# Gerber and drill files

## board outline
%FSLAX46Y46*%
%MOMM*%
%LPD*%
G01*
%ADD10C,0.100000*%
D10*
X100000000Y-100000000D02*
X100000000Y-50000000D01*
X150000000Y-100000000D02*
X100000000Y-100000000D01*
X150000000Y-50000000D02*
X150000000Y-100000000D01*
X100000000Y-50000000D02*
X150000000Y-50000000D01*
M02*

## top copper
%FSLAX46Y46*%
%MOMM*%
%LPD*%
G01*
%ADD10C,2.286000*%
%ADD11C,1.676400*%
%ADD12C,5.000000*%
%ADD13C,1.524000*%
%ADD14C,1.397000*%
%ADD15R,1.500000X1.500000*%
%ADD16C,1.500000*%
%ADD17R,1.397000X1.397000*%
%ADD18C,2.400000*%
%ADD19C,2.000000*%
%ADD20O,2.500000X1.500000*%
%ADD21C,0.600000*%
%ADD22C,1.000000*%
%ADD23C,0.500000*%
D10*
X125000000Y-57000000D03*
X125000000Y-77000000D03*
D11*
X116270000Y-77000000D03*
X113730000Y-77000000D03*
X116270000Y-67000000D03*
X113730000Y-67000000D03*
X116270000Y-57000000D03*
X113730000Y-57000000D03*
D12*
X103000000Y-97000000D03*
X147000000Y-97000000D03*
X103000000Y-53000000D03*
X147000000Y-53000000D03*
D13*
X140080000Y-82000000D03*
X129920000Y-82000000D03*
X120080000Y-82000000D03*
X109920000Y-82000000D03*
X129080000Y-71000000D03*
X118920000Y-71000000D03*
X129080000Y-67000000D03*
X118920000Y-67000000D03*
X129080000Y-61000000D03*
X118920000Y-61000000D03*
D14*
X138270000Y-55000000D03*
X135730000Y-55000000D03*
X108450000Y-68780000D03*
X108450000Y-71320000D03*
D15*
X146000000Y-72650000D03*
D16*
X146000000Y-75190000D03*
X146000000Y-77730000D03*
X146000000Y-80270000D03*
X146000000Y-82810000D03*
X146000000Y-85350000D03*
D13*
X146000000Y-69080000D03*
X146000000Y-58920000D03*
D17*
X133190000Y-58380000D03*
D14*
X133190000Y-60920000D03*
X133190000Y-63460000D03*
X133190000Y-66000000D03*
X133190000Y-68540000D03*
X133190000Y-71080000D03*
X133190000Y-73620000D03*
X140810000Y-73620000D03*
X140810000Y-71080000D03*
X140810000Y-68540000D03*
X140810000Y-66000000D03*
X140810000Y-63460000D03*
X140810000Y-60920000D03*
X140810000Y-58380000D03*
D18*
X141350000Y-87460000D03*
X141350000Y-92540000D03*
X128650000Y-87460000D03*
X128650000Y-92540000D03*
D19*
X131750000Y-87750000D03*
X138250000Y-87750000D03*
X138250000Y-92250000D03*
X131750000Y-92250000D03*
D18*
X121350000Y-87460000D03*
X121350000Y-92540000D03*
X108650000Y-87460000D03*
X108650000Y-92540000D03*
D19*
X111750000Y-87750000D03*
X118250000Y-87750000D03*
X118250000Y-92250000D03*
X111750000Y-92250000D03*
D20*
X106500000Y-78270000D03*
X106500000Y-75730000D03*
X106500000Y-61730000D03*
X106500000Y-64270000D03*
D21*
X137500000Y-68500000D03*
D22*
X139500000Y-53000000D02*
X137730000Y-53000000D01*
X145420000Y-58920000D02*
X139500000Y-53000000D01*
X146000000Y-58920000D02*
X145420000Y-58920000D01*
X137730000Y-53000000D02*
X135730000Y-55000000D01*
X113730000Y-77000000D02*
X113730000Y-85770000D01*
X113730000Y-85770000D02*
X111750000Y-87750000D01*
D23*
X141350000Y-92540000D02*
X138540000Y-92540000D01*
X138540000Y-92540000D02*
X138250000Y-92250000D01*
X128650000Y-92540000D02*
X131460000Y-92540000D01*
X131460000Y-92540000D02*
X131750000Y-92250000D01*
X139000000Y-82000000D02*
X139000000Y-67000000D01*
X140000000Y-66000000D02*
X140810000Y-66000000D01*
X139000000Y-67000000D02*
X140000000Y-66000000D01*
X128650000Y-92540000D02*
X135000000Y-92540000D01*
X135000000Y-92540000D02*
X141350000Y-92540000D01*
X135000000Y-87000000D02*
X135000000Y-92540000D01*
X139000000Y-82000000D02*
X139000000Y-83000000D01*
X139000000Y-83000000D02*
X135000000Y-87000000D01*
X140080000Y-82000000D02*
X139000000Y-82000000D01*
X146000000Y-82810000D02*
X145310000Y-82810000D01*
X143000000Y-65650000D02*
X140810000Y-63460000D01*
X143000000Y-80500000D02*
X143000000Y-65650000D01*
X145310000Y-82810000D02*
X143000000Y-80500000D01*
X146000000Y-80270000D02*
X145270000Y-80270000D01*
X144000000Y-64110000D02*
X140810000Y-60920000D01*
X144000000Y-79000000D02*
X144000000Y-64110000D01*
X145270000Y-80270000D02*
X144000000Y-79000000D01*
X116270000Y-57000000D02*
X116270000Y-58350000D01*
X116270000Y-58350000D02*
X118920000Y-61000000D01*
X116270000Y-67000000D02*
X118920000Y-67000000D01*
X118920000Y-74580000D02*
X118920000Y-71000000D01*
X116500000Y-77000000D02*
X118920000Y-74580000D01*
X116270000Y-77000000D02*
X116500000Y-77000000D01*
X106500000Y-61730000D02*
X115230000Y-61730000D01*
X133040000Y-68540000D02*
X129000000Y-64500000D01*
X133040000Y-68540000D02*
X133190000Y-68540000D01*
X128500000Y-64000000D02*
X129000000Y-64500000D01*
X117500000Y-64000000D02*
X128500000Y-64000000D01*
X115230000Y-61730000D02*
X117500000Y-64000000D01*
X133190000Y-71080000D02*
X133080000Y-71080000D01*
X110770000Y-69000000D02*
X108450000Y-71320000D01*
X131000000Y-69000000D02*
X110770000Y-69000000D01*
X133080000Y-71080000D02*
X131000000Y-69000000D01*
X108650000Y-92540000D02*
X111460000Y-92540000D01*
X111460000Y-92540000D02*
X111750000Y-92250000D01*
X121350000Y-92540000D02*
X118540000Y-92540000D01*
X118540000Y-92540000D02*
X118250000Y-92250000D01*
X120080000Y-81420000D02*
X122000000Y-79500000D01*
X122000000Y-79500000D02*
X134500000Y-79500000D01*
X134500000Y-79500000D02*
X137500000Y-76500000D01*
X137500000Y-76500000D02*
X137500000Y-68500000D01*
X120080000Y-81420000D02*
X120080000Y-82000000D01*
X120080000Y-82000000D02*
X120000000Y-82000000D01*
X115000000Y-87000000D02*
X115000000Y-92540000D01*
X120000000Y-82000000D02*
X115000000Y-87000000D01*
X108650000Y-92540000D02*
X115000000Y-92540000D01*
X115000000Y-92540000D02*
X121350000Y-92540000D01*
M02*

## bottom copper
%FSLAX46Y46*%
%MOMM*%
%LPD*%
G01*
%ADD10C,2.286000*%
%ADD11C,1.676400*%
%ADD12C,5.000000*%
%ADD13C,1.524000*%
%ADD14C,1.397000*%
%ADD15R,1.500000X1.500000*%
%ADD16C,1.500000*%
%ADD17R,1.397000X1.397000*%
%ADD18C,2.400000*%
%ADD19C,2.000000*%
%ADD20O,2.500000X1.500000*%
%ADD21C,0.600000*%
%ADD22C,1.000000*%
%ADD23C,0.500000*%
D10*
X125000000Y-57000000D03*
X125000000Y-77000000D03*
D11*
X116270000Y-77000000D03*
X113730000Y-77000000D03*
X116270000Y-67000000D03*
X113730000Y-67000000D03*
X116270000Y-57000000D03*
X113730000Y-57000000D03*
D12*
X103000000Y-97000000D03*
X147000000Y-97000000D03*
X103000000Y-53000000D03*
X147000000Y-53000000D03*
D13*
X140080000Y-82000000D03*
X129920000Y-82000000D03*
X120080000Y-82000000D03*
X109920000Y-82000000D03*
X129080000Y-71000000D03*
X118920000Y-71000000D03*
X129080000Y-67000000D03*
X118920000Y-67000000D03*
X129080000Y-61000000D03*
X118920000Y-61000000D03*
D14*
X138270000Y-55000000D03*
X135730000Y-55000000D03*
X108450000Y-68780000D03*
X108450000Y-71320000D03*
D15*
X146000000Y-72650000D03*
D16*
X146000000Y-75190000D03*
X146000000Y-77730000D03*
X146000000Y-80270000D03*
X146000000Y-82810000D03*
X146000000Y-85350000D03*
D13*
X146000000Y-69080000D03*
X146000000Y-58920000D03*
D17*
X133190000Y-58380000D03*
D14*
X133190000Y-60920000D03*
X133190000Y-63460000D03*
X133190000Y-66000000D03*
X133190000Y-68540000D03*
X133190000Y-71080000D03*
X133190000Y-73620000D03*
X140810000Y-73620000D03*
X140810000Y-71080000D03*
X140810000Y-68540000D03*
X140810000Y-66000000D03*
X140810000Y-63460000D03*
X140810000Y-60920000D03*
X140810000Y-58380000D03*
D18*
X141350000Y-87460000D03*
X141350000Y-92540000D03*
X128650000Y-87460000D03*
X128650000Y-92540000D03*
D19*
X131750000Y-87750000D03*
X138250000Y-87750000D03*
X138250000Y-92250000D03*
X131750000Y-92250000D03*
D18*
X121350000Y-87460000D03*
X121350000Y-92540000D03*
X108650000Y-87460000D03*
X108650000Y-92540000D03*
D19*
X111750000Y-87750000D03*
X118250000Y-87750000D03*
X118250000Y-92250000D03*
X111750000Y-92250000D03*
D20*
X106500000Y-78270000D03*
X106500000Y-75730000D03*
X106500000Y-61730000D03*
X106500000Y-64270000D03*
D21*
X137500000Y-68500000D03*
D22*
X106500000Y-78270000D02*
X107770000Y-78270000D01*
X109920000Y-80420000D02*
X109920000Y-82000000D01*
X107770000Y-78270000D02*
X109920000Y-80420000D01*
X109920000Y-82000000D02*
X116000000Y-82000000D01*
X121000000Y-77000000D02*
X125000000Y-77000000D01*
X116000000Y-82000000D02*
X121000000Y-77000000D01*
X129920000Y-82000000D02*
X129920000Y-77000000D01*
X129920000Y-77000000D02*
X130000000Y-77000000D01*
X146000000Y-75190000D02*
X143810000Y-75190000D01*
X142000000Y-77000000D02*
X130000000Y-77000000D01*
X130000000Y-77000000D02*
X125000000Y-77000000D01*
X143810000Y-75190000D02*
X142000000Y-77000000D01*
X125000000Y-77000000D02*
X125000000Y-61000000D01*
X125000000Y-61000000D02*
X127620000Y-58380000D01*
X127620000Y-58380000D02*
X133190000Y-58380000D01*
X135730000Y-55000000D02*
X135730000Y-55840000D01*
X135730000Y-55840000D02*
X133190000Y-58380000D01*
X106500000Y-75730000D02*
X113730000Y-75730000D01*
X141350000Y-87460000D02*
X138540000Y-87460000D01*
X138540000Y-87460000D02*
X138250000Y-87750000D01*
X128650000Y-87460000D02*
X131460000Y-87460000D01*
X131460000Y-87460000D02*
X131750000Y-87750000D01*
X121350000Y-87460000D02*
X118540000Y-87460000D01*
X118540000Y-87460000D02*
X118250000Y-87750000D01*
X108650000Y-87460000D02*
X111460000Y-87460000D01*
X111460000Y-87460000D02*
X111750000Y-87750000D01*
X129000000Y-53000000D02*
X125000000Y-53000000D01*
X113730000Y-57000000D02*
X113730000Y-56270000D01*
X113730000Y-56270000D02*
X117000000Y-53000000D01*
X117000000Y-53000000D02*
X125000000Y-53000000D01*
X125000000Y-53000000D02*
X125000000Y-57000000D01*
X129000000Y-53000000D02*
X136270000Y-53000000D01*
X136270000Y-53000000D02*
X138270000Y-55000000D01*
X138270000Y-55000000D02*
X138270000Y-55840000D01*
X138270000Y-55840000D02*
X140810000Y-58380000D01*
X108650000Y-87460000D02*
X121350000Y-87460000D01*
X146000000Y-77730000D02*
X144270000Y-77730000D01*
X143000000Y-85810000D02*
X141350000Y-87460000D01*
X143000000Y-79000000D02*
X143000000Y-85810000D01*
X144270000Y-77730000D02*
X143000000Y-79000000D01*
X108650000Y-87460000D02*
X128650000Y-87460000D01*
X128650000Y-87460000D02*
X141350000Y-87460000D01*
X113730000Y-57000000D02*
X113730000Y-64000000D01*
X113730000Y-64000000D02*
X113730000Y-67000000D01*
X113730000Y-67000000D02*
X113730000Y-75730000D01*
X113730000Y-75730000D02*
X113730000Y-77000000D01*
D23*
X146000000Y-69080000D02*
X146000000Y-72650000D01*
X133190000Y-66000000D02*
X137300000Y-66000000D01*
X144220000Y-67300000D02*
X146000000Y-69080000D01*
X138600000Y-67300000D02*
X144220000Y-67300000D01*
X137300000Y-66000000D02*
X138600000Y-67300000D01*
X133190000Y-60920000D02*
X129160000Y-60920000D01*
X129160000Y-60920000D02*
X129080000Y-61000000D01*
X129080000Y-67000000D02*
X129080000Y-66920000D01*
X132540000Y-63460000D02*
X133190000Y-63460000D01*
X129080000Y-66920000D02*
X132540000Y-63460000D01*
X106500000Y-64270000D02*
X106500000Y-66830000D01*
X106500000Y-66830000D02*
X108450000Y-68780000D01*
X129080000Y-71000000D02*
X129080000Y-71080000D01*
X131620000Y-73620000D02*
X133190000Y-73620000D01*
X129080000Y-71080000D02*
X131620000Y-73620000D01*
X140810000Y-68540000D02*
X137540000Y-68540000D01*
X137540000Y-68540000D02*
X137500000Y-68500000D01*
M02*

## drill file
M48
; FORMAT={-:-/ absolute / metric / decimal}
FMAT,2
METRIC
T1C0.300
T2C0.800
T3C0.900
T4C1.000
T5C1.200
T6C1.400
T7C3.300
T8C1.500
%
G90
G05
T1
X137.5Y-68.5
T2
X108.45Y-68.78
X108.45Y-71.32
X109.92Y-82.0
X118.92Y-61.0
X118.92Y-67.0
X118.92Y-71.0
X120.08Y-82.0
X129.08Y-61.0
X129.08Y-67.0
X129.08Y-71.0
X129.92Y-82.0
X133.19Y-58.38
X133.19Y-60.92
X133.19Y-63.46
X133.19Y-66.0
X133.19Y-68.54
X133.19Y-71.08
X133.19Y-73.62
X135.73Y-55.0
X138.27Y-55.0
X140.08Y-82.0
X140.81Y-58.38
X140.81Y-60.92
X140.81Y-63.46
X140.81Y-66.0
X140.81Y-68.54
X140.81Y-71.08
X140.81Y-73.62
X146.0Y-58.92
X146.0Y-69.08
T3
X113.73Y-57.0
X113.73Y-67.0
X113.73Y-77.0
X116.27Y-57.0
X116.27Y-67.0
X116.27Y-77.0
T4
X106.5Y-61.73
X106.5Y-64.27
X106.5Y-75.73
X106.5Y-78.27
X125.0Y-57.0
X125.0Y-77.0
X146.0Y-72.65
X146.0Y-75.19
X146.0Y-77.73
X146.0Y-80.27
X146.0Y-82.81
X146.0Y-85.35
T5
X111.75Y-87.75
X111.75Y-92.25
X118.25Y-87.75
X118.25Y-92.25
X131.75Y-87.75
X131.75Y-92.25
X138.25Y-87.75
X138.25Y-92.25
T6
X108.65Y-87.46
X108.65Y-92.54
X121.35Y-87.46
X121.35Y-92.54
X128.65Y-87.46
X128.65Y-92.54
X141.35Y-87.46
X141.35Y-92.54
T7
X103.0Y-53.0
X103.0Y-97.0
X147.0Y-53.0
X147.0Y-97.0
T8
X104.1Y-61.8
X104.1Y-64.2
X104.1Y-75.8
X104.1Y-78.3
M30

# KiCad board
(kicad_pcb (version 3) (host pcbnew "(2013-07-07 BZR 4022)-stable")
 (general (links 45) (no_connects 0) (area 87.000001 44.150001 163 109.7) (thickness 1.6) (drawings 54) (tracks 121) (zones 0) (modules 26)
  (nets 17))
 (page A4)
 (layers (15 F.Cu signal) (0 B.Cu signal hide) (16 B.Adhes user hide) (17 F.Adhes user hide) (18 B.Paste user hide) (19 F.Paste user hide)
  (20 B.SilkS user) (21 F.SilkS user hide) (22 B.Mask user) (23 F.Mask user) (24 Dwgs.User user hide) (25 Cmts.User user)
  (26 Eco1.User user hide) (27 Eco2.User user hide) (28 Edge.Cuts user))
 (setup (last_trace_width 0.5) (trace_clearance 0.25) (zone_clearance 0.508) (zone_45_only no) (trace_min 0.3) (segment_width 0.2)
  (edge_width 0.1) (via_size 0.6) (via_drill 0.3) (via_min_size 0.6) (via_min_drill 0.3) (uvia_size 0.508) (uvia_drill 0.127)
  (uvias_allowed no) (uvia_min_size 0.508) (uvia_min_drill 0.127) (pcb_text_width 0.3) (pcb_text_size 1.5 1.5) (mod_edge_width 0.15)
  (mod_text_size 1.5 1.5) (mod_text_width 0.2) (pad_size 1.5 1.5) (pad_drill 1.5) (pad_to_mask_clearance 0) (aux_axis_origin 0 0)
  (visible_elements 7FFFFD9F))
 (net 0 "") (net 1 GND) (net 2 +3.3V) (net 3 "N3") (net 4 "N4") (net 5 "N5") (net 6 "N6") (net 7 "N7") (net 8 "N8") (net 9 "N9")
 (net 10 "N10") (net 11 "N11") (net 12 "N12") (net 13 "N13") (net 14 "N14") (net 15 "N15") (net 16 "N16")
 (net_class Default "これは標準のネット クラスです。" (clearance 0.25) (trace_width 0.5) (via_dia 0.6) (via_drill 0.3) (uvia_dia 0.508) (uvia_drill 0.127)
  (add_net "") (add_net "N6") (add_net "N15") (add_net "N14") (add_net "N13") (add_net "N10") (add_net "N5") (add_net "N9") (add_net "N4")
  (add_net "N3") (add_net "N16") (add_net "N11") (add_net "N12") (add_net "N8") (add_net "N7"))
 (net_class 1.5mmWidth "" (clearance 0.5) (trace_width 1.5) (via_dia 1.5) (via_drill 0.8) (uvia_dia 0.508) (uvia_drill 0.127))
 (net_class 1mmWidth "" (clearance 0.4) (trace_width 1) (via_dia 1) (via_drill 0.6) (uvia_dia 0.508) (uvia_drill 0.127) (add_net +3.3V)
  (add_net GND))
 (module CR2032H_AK (layer B.Cu) (at 125 62 270)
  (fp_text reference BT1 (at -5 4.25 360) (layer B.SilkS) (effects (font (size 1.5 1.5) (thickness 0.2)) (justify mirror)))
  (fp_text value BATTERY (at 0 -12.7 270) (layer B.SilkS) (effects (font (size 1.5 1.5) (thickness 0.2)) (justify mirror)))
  (pad 2 thru_hole circle (at -5 0 270) (size 2.286 2.286) (drill 1) (layers *.Cu *.Mask B.SilkS) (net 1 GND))
  (pad 1 thru_hole circle (at 15 0 270) (size 2.286 2.286) (drill 1) (layers *.Cu *.Mask B.SilkS) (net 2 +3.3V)))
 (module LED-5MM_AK (layer F.Cu) (at 115 77 180)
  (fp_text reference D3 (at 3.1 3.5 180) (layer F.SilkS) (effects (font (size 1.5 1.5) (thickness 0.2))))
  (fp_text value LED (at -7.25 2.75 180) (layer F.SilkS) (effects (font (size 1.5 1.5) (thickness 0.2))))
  (pad 1 thru_hole circle (at -1.27 0 180) (size 1.6764 1.6764) (drill 0.9) (layers *.Cu *.Mask F.SilkS) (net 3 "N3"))
  (pad 2 thru_hole circle (at 1.27 0 180) (size 1.6764 1.6764) (drill 0.9) (layers *.Cu *.Mask F.SilkS) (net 1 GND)))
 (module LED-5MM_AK (layer F.Cu) (at 115 67 180)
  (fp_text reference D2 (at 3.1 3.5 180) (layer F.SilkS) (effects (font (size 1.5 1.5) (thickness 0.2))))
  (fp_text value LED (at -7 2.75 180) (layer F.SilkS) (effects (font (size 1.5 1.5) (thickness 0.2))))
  (pad 1 thru_hole circle (at -1.27 0 180) (size 1.6764 1.6764) (drill 0.9) (layers *.Cu *.Mask F.SilkS) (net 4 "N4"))
  (pad 2 thru_hole circle (at 1.27 0 180) (size 1.6764 1.6764) (drill 0.9) (layers *.Cu *.Mask F.SilkS) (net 1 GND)))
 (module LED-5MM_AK (layer F.Cu) (at 115 57 180)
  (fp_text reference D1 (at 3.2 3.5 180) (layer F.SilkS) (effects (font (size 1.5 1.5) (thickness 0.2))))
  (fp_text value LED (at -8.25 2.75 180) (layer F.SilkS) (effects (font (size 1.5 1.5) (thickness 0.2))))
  (pad 1 thru_hole circle (at -1.27 0 180) (size 1.6764 1.6764) (drill 0.9) (layers *.Cu *.Mask F.SilkS) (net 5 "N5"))
  (pad 2 thru_hole circle (at 1.27 0 180) (size 1.6764 1.6764) (drill 0.9) (layers *.Cu *.Mask F.SilkS) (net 1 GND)))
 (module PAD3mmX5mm (layer F.Cu) (at 103 97)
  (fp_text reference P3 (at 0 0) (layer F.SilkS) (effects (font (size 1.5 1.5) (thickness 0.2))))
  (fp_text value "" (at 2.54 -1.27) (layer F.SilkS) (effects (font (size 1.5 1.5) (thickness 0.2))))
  (pad "" thru_hole circle (at 0 0) (size 5 5) (drill 3.3) (layers *.Cu *.Mask F.SilkS)))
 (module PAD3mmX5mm (layer F.Cu) (at 147 97)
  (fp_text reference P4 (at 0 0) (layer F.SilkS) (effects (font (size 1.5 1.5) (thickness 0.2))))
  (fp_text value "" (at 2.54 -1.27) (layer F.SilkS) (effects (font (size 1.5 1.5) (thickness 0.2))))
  (pad "" thru_hole circle (at 0 0) (size 5 5) (drill 3.3) (layers *.Cu *.Mask F.SilkS)))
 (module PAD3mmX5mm (layer F.Cu) (at 103 53)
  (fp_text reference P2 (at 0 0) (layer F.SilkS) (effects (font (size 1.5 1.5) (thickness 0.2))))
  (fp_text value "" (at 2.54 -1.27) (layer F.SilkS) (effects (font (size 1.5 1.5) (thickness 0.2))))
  (pad "" thru_hole circle (at 0 0) (size 5 5) (drill 3.3) (layers *.Cu *.Mask F.SilkS)))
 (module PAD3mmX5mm (layer F.Cu) (at 147 53)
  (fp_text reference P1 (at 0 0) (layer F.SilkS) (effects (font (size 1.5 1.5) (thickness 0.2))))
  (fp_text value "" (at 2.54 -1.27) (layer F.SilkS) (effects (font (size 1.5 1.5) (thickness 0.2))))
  (pad "" thru_hole circle (at 0 0) (size 5 5) (drill 3.3) (layers *.Cu *.Mask F.SilkS)))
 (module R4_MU (layer F.Cu) (at 135 82 180) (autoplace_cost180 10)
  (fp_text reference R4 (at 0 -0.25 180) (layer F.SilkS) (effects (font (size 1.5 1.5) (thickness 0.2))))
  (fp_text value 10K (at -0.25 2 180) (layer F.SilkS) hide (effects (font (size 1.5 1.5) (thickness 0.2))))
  (pad 1 thru_hole circle (at -5.08 0 180) (size 1.524 1.524) (drill 0.8) (layers *.Cu *.Mask F.SilkS) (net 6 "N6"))
  (pad 2 thru_hole circle (at 5.08 0 180) (size 1.524 1.524) (drill 0.8) (layers *.Cu *.Mask F.SilkS) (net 2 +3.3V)))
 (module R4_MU (layer F.Cu) (at 115 82 180) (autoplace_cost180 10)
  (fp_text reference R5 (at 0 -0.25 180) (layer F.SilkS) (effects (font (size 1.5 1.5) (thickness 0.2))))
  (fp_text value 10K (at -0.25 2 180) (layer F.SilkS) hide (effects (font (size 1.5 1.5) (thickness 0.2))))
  (pad 1 thru_hole circle (at -5.08 0 180) (size 1.524 1.524) (drill 0.8) (layers *.Cu *.Mask F.SilkS) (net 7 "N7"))
  (pad 2 thru_hole circle (at 5.08 0 180) (size 1.524 1.524) (drill 0.8) (layers *.Cu *.Mask F.SilkS) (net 2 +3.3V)))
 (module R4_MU (layer F.Cu) (at 124 71 180) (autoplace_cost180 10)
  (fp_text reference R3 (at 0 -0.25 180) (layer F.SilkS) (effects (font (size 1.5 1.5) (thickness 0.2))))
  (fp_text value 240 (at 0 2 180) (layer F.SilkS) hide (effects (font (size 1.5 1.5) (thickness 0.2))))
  (pad 1 thru_hole circle (at -5.08 0 180) (size 1.524 1.524) (drill 0.8) (layers *.Cu *.Mask F.SilkS) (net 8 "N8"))
  (pad 2 thru_hole circle (at 5.08 0 180) (size 1.524 1.524) (drill 0.8) (layers *.Cu *.Mask F.SilkS) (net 3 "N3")))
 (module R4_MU (layer F.Cu) (at 124 67 180) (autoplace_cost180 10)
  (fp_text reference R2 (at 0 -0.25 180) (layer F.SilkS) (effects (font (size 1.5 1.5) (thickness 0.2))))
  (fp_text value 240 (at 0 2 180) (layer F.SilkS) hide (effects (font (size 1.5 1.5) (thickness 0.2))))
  (pad 1 thru_hole circle (at -5.08 0 180) (size 1.524 1.524) (drill 0.8) (layers *.Cu *.Mask F.SilkS) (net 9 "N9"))
  (pad 2 thru_hole circle (at 5.08 0 180) (size 1.524 1.524) (drill 0.8) (layers *.Cu *.Mask F.SilkS) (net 4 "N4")))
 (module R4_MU (layer F.Cu) (at 124 61 180) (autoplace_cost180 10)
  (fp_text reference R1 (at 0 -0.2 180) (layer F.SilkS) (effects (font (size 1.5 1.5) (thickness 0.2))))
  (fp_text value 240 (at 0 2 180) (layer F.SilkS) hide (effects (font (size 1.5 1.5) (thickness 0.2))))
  (pad 1 thru_hole circle (at -5.08 0 180) (size 1.524 1.524) (drill 0.8) (layers *.Cu *.Mask F.SilkS) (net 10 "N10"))
  (pad 2 thru_hole circle (at 5.08 0 180) (size 1.524 1.524) (drill 0.8) (layers *.Cu *.Mask F.SilkS) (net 5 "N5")))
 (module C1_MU (layer F.Cu) (at 137 55 180)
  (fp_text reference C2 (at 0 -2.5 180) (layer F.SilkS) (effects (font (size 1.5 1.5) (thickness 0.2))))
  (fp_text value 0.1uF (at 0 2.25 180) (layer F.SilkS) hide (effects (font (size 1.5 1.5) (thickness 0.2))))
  (pad 1 thru_hole circle (at -1.27 0 180) (size 1.397 1.397) (drill 0.8) (layers *.Cu *.Mask F.SilkS) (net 1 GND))
  (pad 2 thru_hole circle (at 1.27 0 180) (size 1.397 1.397) (drill 0.8) (layers *.Cu *.Mask F.SilkS) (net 2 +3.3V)))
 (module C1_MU (layer F.Cu) (at 108.45 70.05 270)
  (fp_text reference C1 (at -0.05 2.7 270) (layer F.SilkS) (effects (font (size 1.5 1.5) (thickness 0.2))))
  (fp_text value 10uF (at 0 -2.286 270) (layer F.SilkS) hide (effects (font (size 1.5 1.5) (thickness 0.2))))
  (pad 1 thru_hole circle (at -1.27 0 270) (size 1.397 1.397) (drill 0.8) (layers *.Cu *.Mask F.SilkS) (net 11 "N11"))
  (pad 2 thru_hole circle (at 1.27 0 270) (size 1.397 1.397) (drill 0.8) (layers *.Cu *.Mask F.SilkS) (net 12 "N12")))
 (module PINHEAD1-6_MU (layer F.Cu) (at 146 79 270)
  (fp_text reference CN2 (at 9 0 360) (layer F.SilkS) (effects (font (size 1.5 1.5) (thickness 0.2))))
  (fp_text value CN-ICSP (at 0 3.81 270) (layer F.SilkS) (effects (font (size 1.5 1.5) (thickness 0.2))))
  (pad 1 thru_hole rect (at -6.35 0 270) (size 1.5 1.5) (drill 1) (layers *.Cu *.Mask F.SilkS) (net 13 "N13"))
  (pad 2 thru_hole circle (at -3.81 0 270) (size 1.5 1.5) (drill 1) (layers *.Cu *.Mask F.SilkS) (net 2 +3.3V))
  (pad 3 thru_hole circle (at -1.27 0 270) (size 1.5 1.5) (drill 1) (layers *.Cu *.Mask F.SilkS) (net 1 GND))
  (pad 4 thru_hole circle (at 1.27 0 270) (size 1.5 1.5) (drill 1) (layers *.Cu *.Mask F.SilkS) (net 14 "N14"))
  (pad 5 thru_hole circle (at 3.81 0 270) (size 1.5 1.5) (drill 1) (layers *.Cu *.Mask F.SilkS) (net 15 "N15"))
  (pad 6 thru_hole circle (at 6.35 0 270) (size 1.5 1.5) (drill 1) (layers *.Cu *.Mask F.SilkS)))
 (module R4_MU (layer F.Cu) (at 146 64 90) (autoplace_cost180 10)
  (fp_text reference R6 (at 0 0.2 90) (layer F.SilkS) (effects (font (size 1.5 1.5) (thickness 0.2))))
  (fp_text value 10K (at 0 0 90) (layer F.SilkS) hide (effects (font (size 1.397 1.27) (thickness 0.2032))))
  (pad 1 thru_hole circle (at -5.08 0 90) (size 1.524 1.524) (drill 0.8) (layers *.Cu *.Mask F.SilkS) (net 13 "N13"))
  (pad 2 thru_hole circle (at 5.08 0 90) (size 1.524 1.524) (drill 0.8) (layers *.Cu *.Mask F.SilkS) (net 2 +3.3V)))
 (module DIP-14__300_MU (layer F.Cu) (at 137 66 270)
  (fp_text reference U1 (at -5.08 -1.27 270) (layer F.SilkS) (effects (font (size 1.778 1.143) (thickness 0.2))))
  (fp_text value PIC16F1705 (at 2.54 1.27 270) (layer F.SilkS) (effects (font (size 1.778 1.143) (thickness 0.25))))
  (pad 1 thru_hole rect (at -7.62 3.81 270) (size 1.397 1.397) (drill 0.8) (layers *.Cu *.Mask F.SilkS) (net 2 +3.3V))
  (pad 2 thru_hole circle (at -5.08 3.81 270) (size 1.397 1.397) (drill 0.8) (layers *.Cu *.Mask F.SilkS) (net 10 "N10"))
  (pad 3 thru_hole circle (at -2.54 3.81 270) (size 1.397 1.397) (drill 0.8) (layers *.Cu *.Mask F.SilkS) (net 9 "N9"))
  (pad 4 thru_hole circle (at 0 3.81 270) (size 1.397 1.397) (drill 0.8) (layers *.Cu *.Mask F.SilkS) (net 13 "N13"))
  (pad 5 thru_hole circle (at 2.54 3.81 270) (size 1.397 1.397) (drill 0.8) (layers *.Cu *.Mask F.SilkS) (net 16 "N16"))
  (pad 6 thru_hole circle (at 5.08 3.81 270) (size 1.397 1.397) (drill 0.8) (layers *.Cu *.Mask F.SilkS) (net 12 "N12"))
  (pad 7 thru_hole circle (at 7.62 3.81 270) (size 1.397 1.397) (drill 0.8) (layers *.Cu *.Mask F.SilkS) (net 8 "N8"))
  (pad 8 thru_hole circle (at 7.62 -3.81 270) (size 1.397 1.397) (drill 0.8) (layers *.Cu *.Mask F.SilkS))
  (pad 9 thru_hole circle (at 5.08 -3.81 270) (size 1.397 1.397) (drill 0.8) (layers *.Cu *.Mask F.SilkS))
  (pad 10 thru_hole circle (at 2.54 -3.81 270) (size 1.397 1.397) (drill 0.8) (layers *.Cu *.Mask F.SilkS) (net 7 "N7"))
  (pad 11 thru_hole circle (at 0 -3.81 270) (size 1.397 1.397) (drill 0.8) (layers *.Cu *.Mask F.SilkS) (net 6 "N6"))
  (pad 12 thru_hole circle (at -2.54 -3.81 270) (size 1.397 1.397) (drill 0.8) (layers *.Cu *.Mask F.SilkS) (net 15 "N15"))
  (pad 13 thru_hole circle (at -5.08 -3.81 270) (size 1.397 1.397) (drill 0.8) (layers *.Cu *.Mask F.SilkS) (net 14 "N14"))
  (pad 14 thru_hole circle (at -7.62 -3.81 270) (size 1.397 1.397) (drill 0.8) (layers *.Cu *.Mask F.SilkS) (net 1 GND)))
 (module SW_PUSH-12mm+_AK (layer F.Cu) (at 135 90)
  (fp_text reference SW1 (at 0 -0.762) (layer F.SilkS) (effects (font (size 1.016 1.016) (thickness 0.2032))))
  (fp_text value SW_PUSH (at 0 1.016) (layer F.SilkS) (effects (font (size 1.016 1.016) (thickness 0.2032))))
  (pad 1 thru_hole circle (at 6.35 -2.54) (size 2.4 2.4) (drill 1.4) (layers *.Cu *.Mask F.SilkS) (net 1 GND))
  (pad 2 thru_hole circle (at 6.35 2.54) (size 2.4 2.4) (drill 1.4) (layers *.Cu *.Mask F.SilkS) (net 6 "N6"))
  (pad 1 thru_hole circle (at -6.35 -2.54) (size 2.4 2.4) (drill 1.4) (layers *.Cu *.Mask F.SilkS) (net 1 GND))
  (pad 2 thru_hole circle (at -6.35 2.54) (size 2.4 2.4) (drill 1.4) (layers *.Cu *.Mask F.SilkS) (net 6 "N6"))
  (pad 1 thru_hole circle (at -3.25 -2.25) (size 2 2) (drill 1.2) (layers *.Cu *.Mask F.SilkS) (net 1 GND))
  (pad 1 thru_hole circle (at 3.25 -2.25) (size 2 2) (drill 1.2) (layers *.Cu *.Mask F.SilkS) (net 1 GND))
  (pad 2 thru_hole circle (at 3.25 2.25) (size 2 2) (drill 1.2) (layers *.Cu *.Mask F.SilkS) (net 6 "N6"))
  (pad 2 thru_hole circle (at -3.25 2.25) (size 2 2) (drill 1.2) (layers *.Cu *.Mask F.SilkS) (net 6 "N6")))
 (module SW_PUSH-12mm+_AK (layer F.Cu) (at 115 90)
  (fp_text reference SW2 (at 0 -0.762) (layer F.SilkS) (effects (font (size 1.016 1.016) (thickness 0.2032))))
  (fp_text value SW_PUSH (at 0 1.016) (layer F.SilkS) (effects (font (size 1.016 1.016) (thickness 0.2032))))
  (pad 1 thru_hole circle (at 6.35 -2.54) (size 2.4 2.4) (drill 1.4) (layers *.Cu *.Mask F.SilkS) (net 1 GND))
  (pad 2 thru_hole circle (at 6.35 2.54) (size 2.4 2.4) (drill 1.4) (layers *.Cu *.Mask F.SilkS) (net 7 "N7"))
  (pad 1 thru_hole circle (at -6.35 -2.54) (size 2.4 2.4) (drill 1.4) (layers *.Cu *.Mask F.SilkS) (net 1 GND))
  (pad 2 thru_hole circle (at -6.35 2.54) (size 2.4 2.4) (drill 1.4) (layers *.Cu *.Mask F.SilkS) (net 7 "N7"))
  (pad 1 thru_hole circle (at -3.25 -2.25) (size 2 2) (drill 1.2) (layers *.Cu *.Mask F.SilkS) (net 1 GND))
  (pad 1 thru_hole circle (at 3.25 -2.25) (size 2 2) (drill 1.2) (layers *.Cu *.Mask F.SilkS) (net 1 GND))
  (pad 2 thru_hole circle (at 3.25 2.25) (size 2 2) (drill 1.2) (layers *.Cu *.Mask F.SilkS) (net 7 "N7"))
  (pad 2 thru_hole circle (at -3.25 2.25) (size 2 2) (drill 1.2) (layers *.Cu *.Mask F.SilkS) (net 7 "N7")))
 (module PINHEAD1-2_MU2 (layer B.Cu) (at 106.5 77 90)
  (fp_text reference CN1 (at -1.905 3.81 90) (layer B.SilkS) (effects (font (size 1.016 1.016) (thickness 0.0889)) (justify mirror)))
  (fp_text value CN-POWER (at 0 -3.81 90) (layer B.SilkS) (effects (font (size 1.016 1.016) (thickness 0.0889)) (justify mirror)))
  (pad 1 thru_hole oval (at -1.27 0 90) (size 1.5 2.5) (drill 1) (layers *.Cu *.Mask B.SilkS) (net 2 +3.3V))
  (pad 2 thru_hole oval (at 1.27 0 90) (size 1.5 2.5) (drill 1) (layers *.Cu *.Mask B.SilkS) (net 1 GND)))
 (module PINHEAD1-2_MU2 (layer F.Cu) (at 106.5 63 270)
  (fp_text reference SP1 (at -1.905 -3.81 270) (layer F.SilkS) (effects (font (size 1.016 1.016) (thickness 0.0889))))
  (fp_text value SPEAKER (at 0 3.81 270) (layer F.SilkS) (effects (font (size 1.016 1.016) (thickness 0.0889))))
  (pad 1 thru_hole oval (at -1.27 0 270) (size 1.5 2.5) (drill 1) (layers *.Cu *.Mask F.SilkS) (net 16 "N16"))
  (pad 2 thru_hole oval (at 1.27 0 270) (size 1.5 2.5) (drill 1) (layers *.Cu *.Mask F.SilkS) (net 11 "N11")))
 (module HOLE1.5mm (layer F.Cu) (at 104.1 75.8)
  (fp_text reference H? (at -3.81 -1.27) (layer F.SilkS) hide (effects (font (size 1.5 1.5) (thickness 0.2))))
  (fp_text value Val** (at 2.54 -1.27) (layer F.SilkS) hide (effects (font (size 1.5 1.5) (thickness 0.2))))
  (pad "" np_thru_hole circle (at 0 0) (size 1.5 1.5) (drill 1.5) (layers *.Cu *.Mask F.SilkS) (clearance 0.3)))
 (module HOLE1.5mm (layer F.Cu) (at 104.1 78.3)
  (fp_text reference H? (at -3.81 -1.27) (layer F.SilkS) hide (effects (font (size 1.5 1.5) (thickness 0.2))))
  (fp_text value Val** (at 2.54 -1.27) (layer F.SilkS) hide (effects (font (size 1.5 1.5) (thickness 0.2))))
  (pad "" np_thru_hole circle (at 0 0) (size 1.5 1.5) (drill 1.5) (layers *.Cu *.Mask F.SilkS) (clearance 0.3)))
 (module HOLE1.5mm (layer F.Cu) (at 104.1 61.8)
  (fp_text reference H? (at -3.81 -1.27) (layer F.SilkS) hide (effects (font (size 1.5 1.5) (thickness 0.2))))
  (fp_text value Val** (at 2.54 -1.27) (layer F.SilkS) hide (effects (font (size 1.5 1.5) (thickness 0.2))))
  (pad "" np_thru_hole circle (at 0 0) (size 1.5 1.5) (drill 1.5) (layers *.Cu *.Mask F.SilkS) (clearance 0.3)))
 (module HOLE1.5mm (layer F.Cu) (at 104.1 64.2)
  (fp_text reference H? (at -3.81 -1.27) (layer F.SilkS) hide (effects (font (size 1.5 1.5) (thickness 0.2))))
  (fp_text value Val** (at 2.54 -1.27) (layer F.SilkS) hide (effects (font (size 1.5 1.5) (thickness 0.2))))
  (pad "" np_thru_hole circle (at 0 0) (size 1.5 1.5) (drill 1.5) (layers *.Cu *.Mask F.SilkS) (clearance 0.3)))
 (gr_line (start 100 100) (end 100 50) (angle 90) (layer Edge.Cuts) (width 0.1))
 (gr_line (start 150 100) (end 100 100) (angle 90) (layer Edge.Cuts) (width 0.1))
 (gr_line (start 150 50) (end 150 100) (angle 90) (layer Edge.Cuts) (width 0.1))
 (gr_line (start 100 50) (end 150 50) (angle 90) (layer Edge.Cuts) (width 0.1))
 (segment (start 106.5 78.27) (end 107.77 78.27) (width 1) (layer B.Cu) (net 2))
 (segment (start 109.92 80.42) (end 109.92 82) (width 1) (layer B.Cu) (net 2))
 (segment (start 107.77 78.27) (end 109.92 80.42) (width 1) (layer B.Cu) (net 2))
 (segment (start 139.5 53) (end 137.73 53) (width 1) (layer F.Cu) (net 2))
 (segment (start 145.42 58.92) (end 139.5 53) (width 1) (layer F.Cu) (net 2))
 (segment (start 146 58.92) (end 145.42 58.92) (width 1) (layer F.Cu) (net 2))
 (segment (start 137.73 53) (end 135.73 55) (width 1) (layer F.Cu) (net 2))
 (segment (start 109.92 82) (end 116 82) (width 1) (layer B.Cu) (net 2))
 (segment (start 121 77) (end 125 77) (width 1) (layer B.Cu) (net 2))
 (segment (start 116 82) (end 121 77) (width 1) (layer B.Cu) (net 2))
 (segment (start 129.92 82) (end 129.92 77) (width 1) (layer B.Cu) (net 2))
 (segment (start 129.92 77) (end 130 77) (width 1) (layer B.Cu) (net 2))
 (segment (start 146 75.19) (end 143.81 75.19) (width 1) (layer B.Cu) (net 2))
 (segment (start 142 77) (end 130 77) (width 1) (layer B.Cu) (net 2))
 (segment (start 130 77) (end 125 77) (width 1) (layer B.Cu) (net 2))
 (segment (start 143.81 75.19) (end 142 77) (width 1) (layer B.Cu) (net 2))
 (segment (start 125 77) (end 125 61) (width 1) (layer B.Cu) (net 2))
 (segment (start 125 61) (end 127.62 58.38) (width 1) (layer B.Cu) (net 2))
 (segment (start 127.62 58.38) (end 133.19 58.38) (width 1) (layer B.Cu) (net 2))
 (segment (start 135.73 55) (end 135.73 55.84) (width 1) (layer B.Cu) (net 2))
 (segment (start 135.73 55.84) (end 133.19 58.38) (width 1) (layer B.Cu) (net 2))
 (segment (start 113.73 77) (end 113.73 85.77) (width 1) (layer F.Cu) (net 1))
 (segment (start 113.73 85.77) (end 111.75 87.75) (width 1) (layer F.Cu) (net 1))
 (segment (start 106.5 75.73) (end 113.73 75.73) (width 1) (layer B.Cu) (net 1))
 (segment (start 141.35 87.46) (end 138.54 87.46) (width 1) (layer B.Cu) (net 1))
 (segment (start 138.54 87.46) (end 138.25 87.75) (width 1) (layer B.Cu) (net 1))
 (segment (start 128.65 87.46) (end 131.46 87.46) (width 1) (layer B.Cu) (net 1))
 (segment (start 131.46 87.46) (end 131.75 87.75) (width 1) (layer B.Cu) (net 1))
 (segment (start 121.35 87.46) (end 118.54 87.46) (width 1) (layer B.Cu) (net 1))
 (segment (start 118.54 87.46) (end 118.25 87.75) (width 1) (layer B.Cu) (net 1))
 (segment (start 108.65 87.46) (end 111.46 87.46) (width 1) (layer B.Cu) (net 1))
 (segment (start 111.46 87.46) (end 111.75 87.75) (width 1) (layer B.Cu) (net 1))
 (segment (start 129 53) (end 125 53) (width 1) (layer B.Cu) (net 1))
 (segment (start 113.73 57) (end 113.73 56.27) (width 1) (layer B.Cu) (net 1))
 (segment (start 113.73 56.27) (end 117 53) (width 1) (layer B.Cu) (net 1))
 (segment (start 117 53) (end 125 53) (width 1) (layer B.Cu) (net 1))
 (segment (start 125 53) (end 125 57) (width 1) (layer B.Cu) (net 1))
 (segment (start 129 53) (end 136.27 53) (width 1) (layer B.Cu) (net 1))
 (segment (start 136.27 53) (end 138.27 55) (width 1) (layer B.Cu) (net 1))
 (segment (start 138.27 55) (end 138.27 55.84) (width 1) (layer B.Cu) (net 1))
 (segment (start 138.27 55.84) (end 140.81 58.38) (width 1) (layer B.Cu) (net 1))
 (segment (start 108.65 87.46) (end 121.35 87.46) (width 1) (layer B.Cu) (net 1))
 (segment (start 146 77.73) (end 144.27 77.73) (width 1) (layer B.Cu) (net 1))
 (segment (start 143 85.81) (end 141.35 87.46) (width 1) (layer B.Cu) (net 1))
 (segment (start 143 79) (end 143 85.81) (width 1) (layer B.Cu) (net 1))
 (segment (start 144.27 77.73) (end 143 79) (width 1) (layer B.Cu) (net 1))
 (segment (start 108.65 87.46) (end 128.65 87.46) (width 1) (layer B.Cu) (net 1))
 (segment (start 128.65 87.46) (end 141.35 87.46) (width 1) (layer B.Cu) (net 1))
 (segment (start 113.73 57) (end 113.73 64) (width 1) (layer B.Cu) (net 1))
 (segment (start 113.73 64) (end 113.73 67) (width 1) (layer B.Cu) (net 1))
 (segment (start 113.73 67) (end 113.73 75.73) (width 1) (layer B.Cu) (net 1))
 (segment (start 113.73 75.73) (end 113.73 77) (width 1) (layer B.Cu) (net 1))
 (segment (start 141.35 92.54) (end 138.54 92.54) (width 0.5) (layer F.Cu) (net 6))
 (segment (start 138.54 92.54) (end 138.25 92.25) (width 0.5) (layer F.Cu) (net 6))
 (segment (start 128.65 92.54) (end 131.46 92.54) (width 0.5) (layer F.Cu) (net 6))
 (segment (start 131.46 92.54) (end 131.75 92.25) (width 0.5) (layer F.Cu) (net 6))
 (segment (start 139 82) (end 139 67) (width 0.5) (layer F.Cu) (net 6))
 (segment (start 140 66) (end 140.81 66) (width 0.5) (layer F.Cu) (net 6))
 (segment (start 139 67) (end 140 66) (width 0.5) (layer F.Cu) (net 6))
 (segment (start 128.65 92.54) (end 135 92.54) (width 0.5) (layer F.Cu) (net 6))
 (segment (start 135 92.54) (end 141.35 92.54) (width 0.5) (layer F.Cu) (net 6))
 (segment (start 135 87) (end 135 92.54) (width 0.5) (layer F.Cu) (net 6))
 (segment (start 139 82) (end 139 83) (width 0.5) (layer F.Cu) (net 6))
 (segment (start 139 83) (end 135 87) (width 0.5) (layer F.Cu) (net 6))
 (segment (start 140.08 82) (end 139 82) (width 0.5) (layer F.Cu) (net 6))
 (segment (start 146 82.81) (end 145.31 82.81) (width 0.5) (layer F.Cu) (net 15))
 (segment (start 143 65.65) (end 140.81 63.46) (width 0.5) (layer F.Cu) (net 15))
 (segment (start 143 80.5) (end 143 65.65) (width 0.5) (layer F.Cu) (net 15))
 (segment (start 145.31 82.81) (end 143 80.5) (width 0.5) (layer F.Cu) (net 15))
 (segment (start 146 80.27) (end 145.27 80.27) (width 0.5) (layer F.Cu) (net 14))
 (segment (start 144 64.11) (end 140.81 60.92) (width 0.5) (layer F.Cu) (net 14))
 (segment (start 144 79) (end 144 64.11) (width 0.5) (layer F.Cu) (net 14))
 (segment (start 145.27 80.27) (end 144 79) (width 0.5) (layer F.Cu) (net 14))
 (segment (start 146 69.08) (end 146 72.65) (width 0.5) (layer B.Cu) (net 13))
 (segment (start 133.19 66) (end 137.3 66) (width 0.5) (layer B.Cu) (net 13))
 (segment (start 144.22 67.3) (end 146 69.08) (width 0.5) (layer B.Cu) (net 13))
 (segment (start 138.6 67.3) (end 144.22 67.3) (width 0.5) (layer B.Cu) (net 13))
 (segment (start 137.3 66) (end 138.6 67.3) (width 0.5) (layer B.Cu) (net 13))
 (segment (start 133.19 60.92) (end 129.16 60.92) (width 0.5) (layer B.Cu) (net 10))
 (segment (start 129.16 60.92) (end 129.08 61) (width 0.5) (layer B.Cu) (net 10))
 (segment (start 116.27 57) (end 116.27 58.35) (width 0.5) (layer F.Cu) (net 5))
 (segment (start 116.27 58.35) (end 118.92 61) (width 0.5) (layer F.Cu) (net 5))
 (segment (start 129.08 67) (end 129.08 66.92) (width 0.5) (layer B.Cu) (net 9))
 (segment (start 132.54 63.46) (end 133.19 63.46) (width 0.5) (layer B.Cu) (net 9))
 (segment (start 129.08 66.92) (end 132.54 63.46) (width 0.5) (layer B.Cu) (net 9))
 (segment (start 116.27 67) (end 118.92 67) (width 0.5) (layer F.Cu) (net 4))
 (segment (start 118.92 74.58) (end 118.92 71) (width 0.5) (layer F.Cu) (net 3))
 (segment (start 116.5 77) (end 118.92 74.58) (width 0.5) (layer F.Cu) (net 3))
 (segment (start 116.27 77) (end 116.5 77) (width 0.5) (layer F.Cu) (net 3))
 (segment (start 106.5 61.73) (end 115.23 61.73) (width 0.5) (layer F.Cu) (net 16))
 (segment (start 133.04 68.54) (end 129 64.5) (width 0.5) (layer F.Cu) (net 16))
 (segment (start 133.04 68.54) (end 133.19 68.54) (width 0.5) (layer F.Cu) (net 16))
 (segment (start 128.5 64) (end 129 64.5) (width 0.5) (layer F.Cu) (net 16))
 (segment (start 117.5 64) (end 128.5 64) (width 0.5) (layer F.Cu) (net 16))
 (segment (start 115.23 61.73) (end 117.5 64) (width 0.5) (layer F.Cu) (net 16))
 (segment (start 106.5 64.27) (end 106.5 66.83) (width 0.5) (layer B.Cu) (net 11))
 (segment (start 106.5 66.83) (end 108.45 68.78) (width 0.5) (layer B.Cu) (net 11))
 (segment (start 133.19 71.08) (end 133.08 71.08) (width 0.5) (layer F.Cu) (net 12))
 (segment (start 110.77 69) (end 108.45 71.32) (width 0.5) (layer F.Cu) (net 12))
 (segment (start 131 69) (end 110.77 69) (width 0.5) (layer F.Cu) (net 12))
 (segment (start 133.08 71.08) (end 131 69) (width 0.5) (layer F.Cu) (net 12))
 (segment (start 129.08 71) (end 129.08 71.08) (width 0.5) (layer B.Cu) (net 8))
 (segment (start 131.62 73.62) (end 133.19 73.62) (width 0.5) (layer B.Cu) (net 8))
 (segment (start 129.08 71.08) (end 131.62 73.62) (width 0.5) (layer B.Cu) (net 8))
 (segment (start 108.65 92.54) (end 111.46 92.54) (width 0.5) (layer F.Cu) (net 7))
 (segment (start 111.46 92.54) (end 111.75 92.25) (width 0.5) (layer F.Cu) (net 7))
 (segment (start 121.35 92.54) (end 118.54 92.54) (width 0.5) (layer F.Cu) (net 7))
 (segment (start 118.54 92.54) (end 118.25 92.25) (width 0.5) (layer F.Cu) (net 7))
 (segment (start 140.81 68.54) (end 137.54 68.54) (width 0.5) (layer B.Cu) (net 7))
 (segment (start 120.08 81.42) (end 122 79.5) (width 0.5) (layer F.Cu) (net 7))
 (segment (start 122 79.5) (end 134.5 79.5) (width 0.5) (layer F.Cu) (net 7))
 (segment (start 134.5 79.5) (end 137.5 76.5) (width 0.5) (layer F.Cu) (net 7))
 (segment (start 137.5 76.5) (end 137.5 68.5) (width 0.5) (layer F.Cu) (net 7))
 (segment (start 120.08 81.42) (end 120.08 82) (width 0.5) (layer F.Cu) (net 7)) (via (at 137.5 68.5) (size 0.6) (layers F.Cu B.Cu) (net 7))
 (segment (start 137.54 68.54) (end 137.5 68.5) (width 0.5) (layer B.Cu) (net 7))
 (segment (start 120.08 82) (end 120 82) (width 0.5) (layer F.Cu) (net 7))
 (segment (start 115 87) (end 115 92.54) (width 0.5) (layer F.Cu) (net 7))
 (segment (start 120 82) (end 115 87) (width 0.5) (layer F.Cu) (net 7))
 (segment (start 108.65 92.54) (end 115 92.54) (width 0.5) (layer F.Cu) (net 7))
 (segment (start 115 92.54) (end 121.35 92.54) (width 0.5) (layer F.Cu) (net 7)))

